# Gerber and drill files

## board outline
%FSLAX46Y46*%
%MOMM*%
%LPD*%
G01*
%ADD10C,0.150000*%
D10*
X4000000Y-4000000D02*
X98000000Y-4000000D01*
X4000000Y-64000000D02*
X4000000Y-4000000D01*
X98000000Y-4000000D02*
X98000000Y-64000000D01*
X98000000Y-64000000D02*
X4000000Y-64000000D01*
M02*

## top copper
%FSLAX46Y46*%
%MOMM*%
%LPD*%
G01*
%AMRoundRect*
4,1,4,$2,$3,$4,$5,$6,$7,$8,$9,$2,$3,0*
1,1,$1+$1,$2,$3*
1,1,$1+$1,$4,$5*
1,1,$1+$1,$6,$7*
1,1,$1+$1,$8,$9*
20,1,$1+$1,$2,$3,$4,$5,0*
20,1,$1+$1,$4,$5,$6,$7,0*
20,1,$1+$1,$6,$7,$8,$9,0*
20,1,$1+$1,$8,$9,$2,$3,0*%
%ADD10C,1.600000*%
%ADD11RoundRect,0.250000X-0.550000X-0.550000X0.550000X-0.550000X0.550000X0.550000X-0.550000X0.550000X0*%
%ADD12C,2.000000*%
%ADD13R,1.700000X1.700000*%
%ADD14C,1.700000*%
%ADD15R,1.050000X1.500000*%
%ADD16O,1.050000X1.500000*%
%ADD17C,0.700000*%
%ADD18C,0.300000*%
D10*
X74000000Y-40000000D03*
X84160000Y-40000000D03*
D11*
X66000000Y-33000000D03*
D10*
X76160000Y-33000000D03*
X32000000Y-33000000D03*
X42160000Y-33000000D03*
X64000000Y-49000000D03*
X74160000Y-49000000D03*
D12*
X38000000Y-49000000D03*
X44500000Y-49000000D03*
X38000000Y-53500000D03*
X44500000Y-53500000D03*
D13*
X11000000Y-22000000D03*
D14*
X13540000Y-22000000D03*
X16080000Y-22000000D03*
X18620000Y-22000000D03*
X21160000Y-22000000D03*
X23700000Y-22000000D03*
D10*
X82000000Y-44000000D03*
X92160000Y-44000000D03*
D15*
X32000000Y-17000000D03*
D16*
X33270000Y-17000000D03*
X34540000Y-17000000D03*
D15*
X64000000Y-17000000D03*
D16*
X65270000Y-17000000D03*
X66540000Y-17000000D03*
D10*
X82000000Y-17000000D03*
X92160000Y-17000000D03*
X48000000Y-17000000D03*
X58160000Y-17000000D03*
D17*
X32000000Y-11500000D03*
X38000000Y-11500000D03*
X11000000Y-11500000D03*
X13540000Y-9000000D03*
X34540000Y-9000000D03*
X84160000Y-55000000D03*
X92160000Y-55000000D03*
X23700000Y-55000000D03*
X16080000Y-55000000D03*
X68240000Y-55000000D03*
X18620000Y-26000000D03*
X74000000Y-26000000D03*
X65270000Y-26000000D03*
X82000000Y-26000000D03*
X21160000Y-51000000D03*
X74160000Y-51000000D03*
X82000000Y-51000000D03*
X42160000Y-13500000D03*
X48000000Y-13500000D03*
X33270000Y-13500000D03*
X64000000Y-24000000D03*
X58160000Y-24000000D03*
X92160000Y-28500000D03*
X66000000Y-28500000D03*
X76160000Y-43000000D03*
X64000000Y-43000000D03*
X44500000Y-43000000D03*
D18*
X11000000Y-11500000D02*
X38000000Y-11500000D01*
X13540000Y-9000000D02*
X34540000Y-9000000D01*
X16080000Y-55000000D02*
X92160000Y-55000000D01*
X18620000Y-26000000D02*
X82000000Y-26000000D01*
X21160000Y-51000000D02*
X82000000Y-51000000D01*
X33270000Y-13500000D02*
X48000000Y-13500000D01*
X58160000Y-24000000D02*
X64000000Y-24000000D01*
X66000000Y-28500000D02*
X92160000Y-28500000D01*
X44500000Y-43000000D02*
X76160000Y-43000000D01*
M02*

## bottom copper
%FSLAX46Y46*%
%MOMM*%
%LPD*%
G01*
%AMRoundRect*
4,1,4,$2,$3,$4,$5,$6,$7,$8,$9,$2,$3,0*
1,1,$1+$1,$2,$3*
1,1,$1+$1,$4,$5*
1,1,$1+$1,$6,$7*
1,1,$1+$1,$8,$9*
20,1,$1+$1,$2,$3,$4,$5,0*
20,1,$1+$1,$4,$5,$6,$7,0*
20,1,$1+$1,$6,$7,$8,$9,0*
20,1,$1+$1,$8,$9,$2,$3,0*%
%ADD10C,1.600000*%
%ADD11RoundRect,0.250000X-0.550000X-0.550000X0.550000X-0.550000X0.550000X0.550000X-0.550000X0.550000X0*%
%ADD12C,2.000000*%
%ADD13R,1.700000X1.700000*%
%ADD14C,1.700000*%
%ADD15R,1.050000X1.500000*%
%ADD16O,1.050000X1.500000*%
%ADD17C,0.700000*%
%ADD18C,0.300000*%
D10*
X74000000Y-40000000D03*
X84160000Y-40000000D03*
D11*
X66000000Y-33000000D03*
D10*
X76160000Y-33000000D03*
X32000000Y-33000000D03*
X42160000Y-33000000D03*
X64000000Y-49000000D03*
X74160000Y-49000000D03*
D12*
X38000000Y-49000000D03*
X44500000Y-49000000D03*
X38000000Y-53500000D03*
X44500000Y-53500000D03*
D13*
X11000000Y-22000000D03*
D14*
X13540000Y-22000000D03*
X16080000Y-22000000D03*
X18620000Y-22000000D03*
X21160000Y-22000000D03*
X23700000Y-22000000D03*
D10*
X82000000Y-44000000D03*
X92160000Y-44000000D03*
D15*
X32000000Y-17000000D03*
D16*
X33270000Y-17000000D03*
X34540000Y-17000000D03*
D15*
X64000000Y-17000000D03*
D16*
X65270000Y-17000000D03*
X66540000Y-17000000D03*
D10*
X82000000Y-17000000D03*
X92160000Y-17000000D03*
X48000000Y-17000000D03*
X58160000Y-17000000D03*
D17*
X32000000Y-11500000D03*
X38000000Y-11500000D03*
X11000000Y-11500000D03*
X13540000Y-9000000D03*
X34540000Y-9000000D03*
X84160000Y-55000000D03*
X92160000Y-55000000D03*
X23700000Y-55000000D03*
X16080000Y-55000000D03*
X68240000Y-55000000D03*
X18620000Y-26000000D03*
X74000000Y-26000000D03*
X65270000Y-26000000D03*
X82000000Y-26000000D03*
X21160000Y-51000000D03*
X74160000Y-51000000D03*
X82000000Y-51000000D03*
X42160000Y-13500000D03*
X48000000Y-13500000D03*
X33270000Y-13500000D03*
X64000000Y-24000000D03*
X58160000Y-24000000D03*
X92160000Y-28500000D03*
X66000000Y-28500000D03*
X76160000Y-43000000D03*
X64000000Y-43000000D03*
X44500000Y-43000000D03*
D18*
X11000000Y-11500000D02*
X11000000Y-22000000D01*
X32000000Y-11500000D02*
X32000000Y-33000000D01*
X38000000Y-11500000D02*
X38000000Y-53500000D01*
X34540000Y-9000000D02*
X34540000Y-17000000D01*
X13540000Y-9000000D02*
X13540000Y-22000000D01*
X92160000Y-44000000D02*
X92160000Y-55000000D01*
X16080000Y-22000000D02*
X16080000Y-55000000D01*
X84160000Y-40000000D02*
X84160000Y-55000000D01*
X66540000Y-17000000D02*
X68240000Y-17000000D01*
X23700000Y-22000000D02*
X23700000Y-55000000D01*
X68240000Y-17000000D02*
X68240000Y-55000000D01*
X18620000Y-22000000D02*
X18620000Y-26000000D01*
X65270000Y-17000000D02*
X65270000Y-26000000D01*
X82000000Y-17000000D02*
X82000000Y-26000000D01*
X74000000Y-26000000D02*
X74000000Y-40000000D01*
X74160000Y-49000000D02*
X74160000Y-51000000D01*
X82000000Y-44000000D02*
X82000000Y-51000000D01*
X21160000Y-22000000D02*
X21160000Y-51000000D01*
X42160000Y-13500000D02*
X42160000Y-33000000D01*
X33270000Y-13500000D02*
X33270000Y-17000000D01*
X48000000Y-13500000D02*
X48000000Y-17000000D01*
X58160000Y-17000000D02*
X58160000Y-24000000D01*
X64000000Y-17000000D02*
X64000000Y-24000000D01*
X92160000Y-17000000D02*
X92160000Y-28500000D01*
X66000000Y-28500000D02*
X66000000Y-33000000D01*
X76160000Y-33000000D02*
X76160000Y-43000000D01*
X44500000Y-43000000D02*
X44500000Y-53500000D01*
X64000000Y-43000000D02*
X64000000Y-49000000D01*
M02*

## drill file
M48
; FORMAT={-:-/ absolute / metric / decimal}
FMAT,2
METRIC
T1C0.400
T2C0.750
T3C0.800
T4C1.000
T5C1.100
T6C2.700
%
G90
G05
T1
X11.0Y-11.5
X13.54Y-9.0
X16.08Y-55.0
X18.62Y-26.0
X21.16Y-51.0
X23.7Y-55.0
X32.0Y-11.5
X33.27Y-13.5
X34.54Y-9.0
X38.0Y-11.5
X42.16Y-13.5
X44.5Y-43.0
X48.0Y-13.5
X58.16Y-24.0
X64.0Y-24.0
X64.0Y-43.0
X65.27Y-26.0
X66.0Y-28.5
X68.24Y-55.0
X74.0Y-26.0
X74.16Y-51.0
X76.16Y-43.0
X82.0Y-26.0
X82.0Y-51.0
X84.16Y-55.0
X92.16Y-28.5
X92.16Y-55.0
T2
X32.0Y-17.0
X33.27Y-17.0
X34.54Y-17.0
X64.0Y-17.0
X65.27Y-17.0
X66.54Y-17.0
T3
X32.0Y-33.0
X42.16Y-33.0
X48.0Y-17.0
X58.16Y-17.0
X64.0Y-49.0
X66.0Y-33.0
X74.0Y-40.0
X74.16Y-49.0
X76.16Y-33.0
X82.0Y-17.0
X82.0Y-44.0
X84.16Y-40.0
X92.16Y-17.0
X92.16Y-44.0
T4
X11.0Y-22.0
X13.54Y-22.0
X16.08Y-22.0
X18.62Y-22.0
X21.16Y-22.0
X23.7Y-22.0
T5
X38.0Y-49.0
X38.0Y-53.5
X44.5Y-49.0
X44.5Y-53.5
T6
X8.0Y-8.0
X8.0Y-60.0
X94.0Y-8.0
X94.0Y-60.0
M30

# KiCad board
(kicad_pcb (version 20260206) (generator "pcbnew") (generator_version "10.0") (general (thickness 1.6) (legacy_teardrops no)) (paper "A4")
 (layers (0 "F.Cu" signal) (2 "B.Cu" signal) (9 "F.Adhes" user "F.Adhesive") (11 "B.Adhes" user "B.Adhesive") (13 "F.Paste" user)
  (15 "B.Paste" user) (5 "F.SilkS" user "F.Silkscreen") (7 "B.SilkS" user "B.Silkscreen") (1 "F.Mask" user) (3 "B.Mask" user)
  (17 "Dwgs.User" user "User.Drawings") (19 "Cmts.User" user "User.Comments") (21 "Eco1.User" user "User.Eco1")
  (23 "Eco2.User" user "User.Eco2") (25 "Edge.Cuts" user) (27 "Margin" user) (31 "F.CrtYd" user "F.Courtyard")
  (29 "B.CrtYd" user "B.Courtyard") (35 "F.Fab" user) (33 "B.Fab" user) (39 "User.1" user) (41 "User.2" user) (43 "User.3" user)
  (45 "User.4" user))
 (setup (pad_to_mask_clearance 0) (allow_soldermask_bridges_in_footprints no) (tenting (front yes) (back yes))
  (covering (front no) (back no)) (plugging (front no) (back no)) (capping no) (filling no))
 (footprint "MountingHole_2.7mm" (layer "F.Cu") (at 8 8)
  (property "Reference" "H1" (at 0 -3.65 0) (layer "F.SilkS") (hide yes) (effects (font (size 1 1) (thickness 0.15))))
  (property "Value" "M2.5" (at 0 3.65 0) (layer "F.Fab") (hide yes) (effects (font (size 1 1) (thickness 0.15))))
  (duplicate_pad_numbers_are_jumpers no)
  (pad "" np_thru_hole circle (at 0 0) (size 2.7 2.7) (drill 2.7) (layers "*.Cu" "*.Mask")))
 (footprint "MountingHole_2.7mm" (layer "F.Cu") (at 94 60)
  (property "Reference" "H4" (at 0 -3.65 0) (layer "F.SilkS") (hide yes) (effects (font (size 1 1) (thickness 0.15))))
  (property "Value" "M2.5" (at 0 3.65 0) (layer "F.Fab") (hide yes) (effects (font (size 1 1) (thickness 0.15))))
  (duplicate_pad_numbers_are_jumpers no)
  (pad "" np_thru_hole circle (at 0 0) (size 2.7 2.7) (drill 2.7) (layers "*.Cu" "*.Mask")))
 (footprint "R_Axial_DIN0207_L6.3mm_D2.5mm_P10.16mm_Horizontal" (layer "F.Cu") (at 74 40)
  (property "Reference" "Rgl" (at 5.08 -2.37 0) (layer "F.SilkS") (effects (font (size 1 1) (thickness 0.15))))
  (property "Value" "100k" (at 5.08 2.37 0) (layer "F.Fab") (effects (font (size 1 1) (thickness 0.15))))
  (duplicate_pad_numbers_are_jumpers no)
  (pad "1" thru_hole circle (at 0 0) (size 1.6 1.6) (drill 0.8) (layers "*.Cu" "*.Mask") (remove_unused_layers no) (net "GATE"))
  (pad "2" thru_hole circle (at 10.16 0) (size 1.6 1.6) (drill 0.8) (layers "*.Cu" "*.Mask") (remove_unused_layers no) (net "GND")))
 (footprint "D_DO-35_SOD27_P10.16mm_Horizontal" (layer "F.Cu") (at 66 33)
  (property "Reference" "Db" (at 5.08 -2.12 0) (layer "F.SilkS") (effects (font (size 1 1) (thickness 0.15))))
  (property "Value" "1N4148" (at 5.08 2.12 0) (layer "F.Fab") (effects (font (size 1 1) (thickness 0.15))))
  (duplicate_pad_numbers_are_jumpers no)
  (pad "1" thru_hole roundrect (at 0 0) (size 1.6 1.6) (drill 0.8) (layers "*.Cu" "*.Mask") (remove_unused_layers no)
   (roundrect_rratio 0.15625) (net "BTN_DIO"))
  (pad "2" thru_hole circle (at 10.16 0) (size 1.6 1.6) (drill 0.8) (layers "*.Cu" "*.Mask") (remove_unused_layers no) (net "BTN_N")))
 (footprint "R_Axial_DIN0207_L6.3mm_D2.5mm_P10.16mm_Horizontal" (layer "F.Cu") (at 32 33)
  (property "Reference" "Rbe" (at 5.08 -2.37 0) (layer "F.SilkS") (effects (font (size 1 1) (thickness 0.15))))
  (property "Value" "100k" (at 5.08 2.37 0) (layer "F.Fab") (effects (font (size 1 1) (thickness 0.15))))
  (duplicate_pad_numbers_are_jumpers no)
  (pad "1" thru_hole circle (at 0 0) (size 1.6 1.6) (drill 0.8) (layers "*.Cu" "*.Mask") (remove_unused_layers no) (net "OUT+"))
  (pad "2" thru_hole circle (at 10.16 0) (size 1.6 1.6) (drill 0.8) (layers "*.Cu" "*.Mask") (remove_unused_layers no) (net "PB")))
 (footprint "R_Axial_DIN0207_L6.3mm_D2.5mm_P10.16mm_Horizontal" (layer "F.Cu") (at 64 49)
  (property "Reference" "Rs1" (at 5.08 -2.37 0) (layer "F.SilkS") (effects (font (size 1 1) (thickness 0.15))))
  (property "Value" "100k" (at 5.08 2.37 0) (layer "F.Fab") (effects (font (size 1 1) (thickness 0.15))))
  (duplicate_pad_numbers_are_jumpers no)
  (pad "1" thru_hole circle (at 0 0) (size 1.6 1.6) (drill 0.8) (layers "*.Cu" "*.Mask") (remove_unused_layers no) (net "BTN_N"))
  (pad "2" thru_hole circle (at 10.16 0) (size 1.6 1.6) (drill 0.8) (layers "*.Cu" "*.Mask") (remove_unused_layers no) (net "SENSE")))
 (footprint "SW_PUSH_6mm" (layer "F.Cu") (at 38 49)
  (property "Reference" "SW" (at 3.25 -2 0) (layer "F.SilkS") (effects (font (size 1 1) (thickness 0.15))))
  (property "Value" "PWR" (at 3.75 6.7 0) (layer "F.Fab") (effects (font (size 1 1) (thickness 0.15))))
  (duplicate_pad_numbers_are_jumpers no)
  (pad "1" thru_hole circle (at 0 0 90) (size 2 2) (drill 1.1) (layers "*.Cu" "*.Mask") (remove_unused_layers no) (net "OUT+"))
  (pad "1" thru_hole circle (at 6.5 0 90) (size 2 2) (drill 1.1) (layers "*.Cu" "*.Mask") (remove_unused_layers no) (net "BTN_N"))
  (pad "2" thru_hole circle (at 0 4.5 90) (size 2 2) (drill 1.1) (layers "*.Cu" "*.Mask") (remove_unused_layers no) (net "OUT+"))
  (pad "2" thru_hole circle (at 6.5 4.5 90) (size 2 2) (drill 1.1) (layers "*.Cu" "*.Mask") (remove_unused_layers no) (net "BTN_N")))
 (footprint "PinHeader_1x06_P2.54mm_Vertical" (layer "F.Cu") (at 11 22 90)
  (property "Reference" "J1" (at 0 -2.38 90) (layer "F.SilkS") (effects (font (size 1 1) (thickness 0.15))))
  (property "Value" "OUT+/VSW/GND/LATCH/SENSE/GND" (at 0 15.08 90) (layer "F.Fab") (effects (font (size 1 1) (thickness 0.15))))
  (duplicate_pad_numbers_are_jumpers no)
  (pad "1" thru_hole rect (at 0 0 90) (size 1.7 1.7) (drill 1) (layers "*.Cu" "*.Mask") (remove_unused_layers no) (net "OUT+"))
  (pad "2" thru_hole circle (at 0 2.54 90) (size 1.7 1.7) (drill 1) (layers "*.Cu" "*.Mask") (remove_unused_layers no) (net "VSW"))
  (pad "3" thru_hole circle (at 0 5.08 90) (size 1.7 1.7) (drill 1) (layers "*.Cu" "*.Mask") (remove_unused_layers no) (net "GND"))
  (pad "4" thru_hole circle (at 0 7.62 90) (size 1.7 1.7) (drill 1) (layers "*.Cu" "*.Mask") (remove_unused_layers no) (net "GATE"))
  (pad "5" thru_hole circle (at 0 10.16 90) (size 1.7 1.7) (drill 1) (layers "*.Cu" "*.Mask") (remove_unused_layers no) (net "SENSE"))
  (pad "6" thru_hole circle (at 0 12.7 90) (size 1.7 1.7) (drill 1) (layers "*.Cu" "*.Mask") (remove_unused_layers no) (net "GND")))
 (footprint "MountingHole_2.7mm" (layer "F.Cu") (at 8 60)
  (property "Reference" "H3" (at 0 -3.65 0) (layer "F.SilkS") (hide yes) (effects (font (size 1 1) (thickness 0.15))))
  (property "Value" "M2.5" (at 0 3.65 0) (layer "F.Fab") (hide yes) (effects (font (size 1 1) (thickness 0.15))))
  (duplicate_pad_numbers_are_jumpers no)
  (pad "" np_thru_hole circle (at 0 0) (size 2.7 2.7) (drill 2.7) (layers "*.Cu" "*.Mask")))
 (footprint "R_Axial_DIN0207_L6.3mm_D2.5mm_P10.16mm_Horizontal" (layer "F.Cu") (at 82 44)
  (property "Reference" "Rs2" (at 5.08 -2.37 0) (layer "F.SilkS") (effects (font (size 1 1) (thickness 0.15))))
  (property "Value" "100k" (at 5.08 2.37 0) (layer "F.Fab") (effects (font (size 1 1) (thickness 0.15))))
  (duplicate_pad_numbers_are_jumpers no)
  (pad "1" thru_hole circle (at 0 0) (size 1.6 1.6) (drill 0.8) (layers "*.Cu" "*.Mask") (remove_unused_layers no) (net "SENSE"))
  (pad "2" thru_hole circle (at 10.16 0) (size 1.6 1.6) (drill 0.8) (layers "*.Cu" "*.Mask") (remove_unused_layers no) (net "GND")))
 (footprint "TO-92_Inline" (layer "F.Cu") (at 32 17)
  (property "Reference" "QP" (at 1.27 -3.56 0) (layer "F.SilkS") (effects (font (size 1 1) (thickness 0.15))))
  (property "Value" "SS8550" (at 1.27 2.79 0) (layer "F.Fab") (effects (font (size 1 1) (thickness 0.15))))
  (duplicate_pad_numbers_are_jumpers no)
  (pad "1" thru_hole rect (at 0 0) (size 1.05 1.5) (drill 0.75) (layers "*.Cu" "*.Mask") (remove_unused_layers no) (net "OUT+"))
  (pad "2" thru_hole oval (at 1.27 0) (size 1.05 1.5) (drill 0.75) (layers "*.Cu" "*.Mask") (remove_unused_layers no) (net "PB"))
  (pad "3" thru_hole oval (at 2.54 0) (size 1.05 1.5) (drill 0.75) (layers "*.Cu" "*.Mask") (remove_unused_layers no) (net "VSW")))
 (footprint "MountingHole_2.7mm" (layer "F.Cu") (at 94 8)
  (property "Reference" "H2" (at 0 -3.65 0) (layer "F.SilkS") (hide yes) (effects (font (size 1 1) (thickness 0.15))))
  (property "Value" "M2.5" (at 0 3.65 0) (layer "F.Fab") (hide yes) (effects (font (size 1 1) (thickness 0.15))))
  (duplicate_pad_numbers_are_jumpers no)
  (pad "" np_thru_hole circle (at 0 0) (size 2.7 2.7) (drill 2.7) (layers "*.Cu" "*.Mask")))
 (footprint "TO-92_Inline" (layer "F.Cu") (at 64 17)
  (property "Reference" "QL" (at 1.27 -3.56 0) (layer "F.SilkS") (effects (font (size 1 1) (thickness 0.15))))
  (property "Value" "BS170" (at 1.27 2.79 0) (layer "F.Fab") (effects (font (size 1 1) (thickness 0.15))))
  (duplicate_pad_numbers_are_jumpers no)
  (pad "1" thru_hole rect (at 0 0) (size 1.05 1.5) (drill 0.75) (layers "*.Cu" "*.Mask") (remove_unused_layers no) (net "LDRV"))
  (pad "2" thru_hole oval (at 1.27 0) (size 1.05 1.5) (drill 0.75) (layers "*.Cu" "*.Mask") (remove_unused_layers no) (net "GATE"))
  (pad "3" thru_hole oval (at 2.54 0) (size 1.05 1.5) (drill 0.75) (layers "*.Cu" "*.Mask") (remove_unused_layers no) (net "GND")))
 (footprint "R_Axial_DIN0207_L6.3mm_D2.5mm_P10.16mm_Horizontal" (layer "F.Cu") (at 82 17)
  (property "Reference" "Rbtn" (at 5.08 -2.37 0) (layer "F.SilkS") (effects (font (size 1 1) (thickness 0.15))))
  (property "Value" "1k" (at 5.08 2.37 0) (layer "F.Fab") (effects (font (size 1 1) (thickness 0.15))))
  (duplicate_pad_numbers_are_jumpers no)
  (pad "1" thru_hole circle (at 0 0) (size 1.6 1.6) (drill 0.8) (layers "*.Cu" "*.Mask") (remove_unused_layers no) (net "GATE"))
  (pad "2" thru_hole circle (at 10.16 0) (size 1.6 1.6) (drill 0.8) (layers "*.Cu" "*.Mask") (remove_unused_layers no) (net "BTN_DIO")))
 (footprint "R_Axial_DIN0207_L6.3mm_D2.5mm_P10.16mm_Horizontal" (layer "F.Cu") (at 48 17)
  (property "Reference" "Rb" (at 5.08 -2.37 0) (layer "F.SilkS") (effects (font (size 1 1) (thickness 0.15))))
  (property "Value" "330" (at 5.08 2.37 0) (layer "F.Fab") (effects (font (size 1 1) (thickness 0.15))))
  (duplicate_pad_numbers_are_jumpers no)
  (pad "1" thru_hole circle (at 0 0) (size 1.6 1.6) (drill 0.8) (layers "*.Cu" "*.Mask") (remove_unused_layers no) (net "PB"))
  (pad "2" thru_hole circle (at 10.16 0) (size 1.6 1.6) (drill 0.8) (layers "*.Cu" "*.Mask") (remove_unused_layers no) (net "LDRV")))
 (gr_line (start 4 4) (end 98 4) (stroke (width 0.15) (type default)) (layer "Edge.Cuts"))
 (gr_line (start 4 64) (end 4 4) (stroke (width 0.15) (type default)) (layer "Edge.Cuts"))
 (gr_line (start 98 4) (end 98 64) (stroke (width 0.15) (type default)) (layer "Edge.Cuts"))
 (gr_line (start 98 64) (end 4 64) (stroke (width 0.15) (type default)) (layer "Edge.Cuts"))
 (segment (start 11 11.5) (end 38 11.5) (width 0.3) (layer "F.Cu") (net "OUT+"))
 (via (at 32 11.5) (size 0.7) (drill 0.4) (layers "F.Cu" "B.Cu") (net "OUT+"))
 (via (at 38 11.5) (size 0.7) (drill 0.4) (layers "F.Cu" "B.Cu") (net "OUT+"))
 (via (at 11 11.5) (size 0.7) (drill 0.4) (layers "F.Cu" "B.Cu") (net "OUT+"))
 (segment (start 11 11.5) (end 11 22) (width 0.3) (layer "B.Cu") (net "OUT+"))
 (segment (start 32 11.5) (end 32 33) (width 0.3) (layer "B.Cu") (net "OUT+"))
 (segment (start 38 11.5) (end 38 53.5) (width 0.3) (layer "B.Cu") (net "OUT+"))
 (segment (start 13.54 9) (end 34.54 9) (width 0.3) (layer "F.Cu") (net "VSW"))
 (via (at 13.54 9) (size 0.7) (drill 0.4) (layers "F.Cu" "B.Cu") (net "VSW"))
 (via (at 34.54 9) (size 0.7) (drill 0.4) (layers "F.Cu" "B.Cu") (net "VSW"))
 (segment (start 34.54 9) (end 34.54 17) (width 0.3) (layer "B.Cu") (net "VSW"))
 (segment (start 13.54 9) (end 13.54 22) (width 0.3) (layer "B.Cu") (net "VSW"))
 (segment (start 16.08 55) (end 92.16 55) (width 0.3) (layer "F.Cu") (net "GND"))
 (via (at 84.16 55) (size 0.7) (drill 0.4) (layers "F.Cu" "B.Cu") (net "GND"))
 (via (at 92.16 55) (size 0.7) (drill 0.4) (layers "F.Cu" "B.Cu") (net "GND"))
 (via (at 23.7 55) (size 0.7) (drill 0.4) (layers "F.Cu" "B.Cu") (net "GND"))
 (via (at 16.08 55) (size 0.7) (drill 0.4) (layers "F.Cu" "B.Cu") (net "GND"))
 (via (at 68.24 55) (size 0.7) (drill 0.4) (layers "F.Cu" "B.Cu") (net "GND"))
 (segment (start 92.16 44) (end 92.16 55) (width 0.3) (layer "B.Cu") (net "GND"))
 (segment (start 16.08 22) (end 16.08 55) (width 0.3) (layer "B.Cu") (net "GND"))
 (segment (start 84.16 40) (end 84.16 55) (width 0.3) (layer "B.Cu") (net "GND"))
 (segment (start 66.54 17) (end 68.24 17) (width 0.3) (layer "B.Cu") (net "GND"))
 (segment (start 23.7 22) (end 23.7 55) (width 0.3) (layer "B.Cu") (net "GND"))
 (segment (start 68.24 17) (end 68.24 55) (width 0.3) (layer "B.Cu") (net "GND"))
 (segment (start 18.62 26) (end 82 26) (width 0.3) (layer "F.Cu") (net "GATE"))
 (via (at 18.62 26) (size 0.7) (drill 0.4) (layers "F.Cu" "B.Cu") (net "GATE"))
 (via (at 74 26) (size 0.7) (drill 0.4) (layers "F.Cu" "B.Cu") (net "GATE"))
 (via (at 65.27 26) (size 0.7) (drill 0.4) (layers "F.Cu" "B.Cu") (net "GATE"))
 (via (at 82 26) (size 0.7) (drill 0.4) (layers "F.Cu" "B.Cu") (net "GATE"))
 (segment (start 18.62 22) (end 18.62 26) (width 0.3) (layer "B.Cu") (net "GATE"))
 (segment (start 65.27 17) (end 65.27 26) (width 0.3) (layer "B.Cu") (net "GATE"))
 (segment (start 82 17) (end 82 26) (width 0.3) (layer "B.Cu") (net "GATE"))
 (segment (start 74 26) (end 74 40) (width 0.3) (layer "B.Cu") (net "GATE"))
 (segment (start 21.16 51) (end 82 51) (width 0.3) (layer "F.Cu") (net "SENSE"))
 (via (at 21.16 51) (size 0.7) (drill 0.4) (layers "F.Cu" "B.Cu") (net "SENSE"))
 (via (at 74.16 51) (size 0.7) (drill 0.4) (layers "F.Cu" "B.Cu") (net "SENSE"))
 (via (at 82 51) (size 0.7) (drill 0.4) (layers "F.Cu" "B.Cu") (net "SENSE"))
 (segment (start 74.16 49) (end 74.16 51) (width 0.3) (layer "B.Cu") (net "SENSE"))
 (segment (start 82 44) (end 82 51) (width 0.3) (layer "B.Cu") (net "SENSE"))
 (segment (start 21.16 22) (end 21.16 51) (width 0.3) (layer "B.Cu") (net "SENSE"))
 (segment (start 33.27 13.5) (end 48 13.5) (width 0.3) (layer "F.Cu") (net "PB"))
 (via (at 42.16 13.5) (size 0.7) (drill 0.4) (layers "F.Cu" "B.Cu") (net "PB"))
 (via (at 48 13.5) (size 0.7) (drill 0.4) (layers "F.Cu" "B.Cu") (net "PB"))
 (via (at 33.27 13.5) (size 0.7) (drill 0.4) (layers "F.Cu" "B.Cu") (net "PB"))
 (segment (start 42.16 13.5) (end 42.16 33) (width 0.3) (layer "B.Cu") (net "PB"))
 (segment (start 33.27 13.5) (end 33.27 17) (width 0.3) (layer "B.Cu") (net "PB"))
 (segment (start 48 13.5) (end 48 17) (width 0.3) (layer "B.Cu") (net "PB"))
 (segment (start 58.16 24) (end 64 24) (width 0.3) (layer "F.Cu") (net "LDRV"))
 (via (at 64 24) (size 0.7) (drill 0.4) (layers "F.Cu" "B.Cu") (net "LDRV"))
 (via (at 58.16 24) (size 0.7) (drill 0.4) (layers "F.Cu" "B.Cu") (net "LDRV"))
 (segment (start 58.16 17) (end 58.16 24) (width 0.3) (layer "B.Cu") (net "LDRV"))
 (segment (start 64 17) (end 64 24) (width 0.3) (layer "B.Cu") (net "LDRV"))
 (segment (start 66 28.5) (end 92.16 28.5) (width 0.3) (layer "F.Cu") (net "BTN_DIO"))
 (via (at 92.16 28.5) (size 0.7) (drill 0.4) (layers "F.Cu" "B.Cu") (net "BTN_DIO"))
 (via (at 66 28.5) (size 0.7) (drill 0.4) (layers "F.Cu" "B.Cu") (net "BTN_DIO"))
 (segment (start 92.16 17) (end 92.16 28.5) (width 0.3) (layer "B.Cu") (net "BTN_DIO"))
 (segment (start 66 28.5) (end 66 33) (width 0.3) (layer "B.Cu") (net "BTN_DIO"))
 (segment (start 44.5 43) (end 76.16 43) (width 0.3) (layer "F.Cu") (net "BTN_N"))
 (via (at 76.16 43) (size 0.7) (drill 0.4) (layers "F.Cu" "B.Cu") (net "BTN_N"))
 (via (at 64 43) (size 0.7) (drill 0.4) (layers "F.Cu" "B.Cu") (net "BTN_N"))
 (via (at 44.5 43) (size 0.7) (drill 0.4) (layers "F.Cu" "B.Cu") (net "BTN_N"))
 (segment (start 76.16 33) (end 76.16 43) (width 0.3) (layer "B.Cu") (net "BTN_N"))
 (segment (start 44.5 43) (end 44.5 53.5) (width 0.3) (layer "B.Cu") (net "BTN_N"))
 (segment (start 64 43) (end 64 49) (width 0.3) (layer "B.Cu") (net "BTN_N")))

